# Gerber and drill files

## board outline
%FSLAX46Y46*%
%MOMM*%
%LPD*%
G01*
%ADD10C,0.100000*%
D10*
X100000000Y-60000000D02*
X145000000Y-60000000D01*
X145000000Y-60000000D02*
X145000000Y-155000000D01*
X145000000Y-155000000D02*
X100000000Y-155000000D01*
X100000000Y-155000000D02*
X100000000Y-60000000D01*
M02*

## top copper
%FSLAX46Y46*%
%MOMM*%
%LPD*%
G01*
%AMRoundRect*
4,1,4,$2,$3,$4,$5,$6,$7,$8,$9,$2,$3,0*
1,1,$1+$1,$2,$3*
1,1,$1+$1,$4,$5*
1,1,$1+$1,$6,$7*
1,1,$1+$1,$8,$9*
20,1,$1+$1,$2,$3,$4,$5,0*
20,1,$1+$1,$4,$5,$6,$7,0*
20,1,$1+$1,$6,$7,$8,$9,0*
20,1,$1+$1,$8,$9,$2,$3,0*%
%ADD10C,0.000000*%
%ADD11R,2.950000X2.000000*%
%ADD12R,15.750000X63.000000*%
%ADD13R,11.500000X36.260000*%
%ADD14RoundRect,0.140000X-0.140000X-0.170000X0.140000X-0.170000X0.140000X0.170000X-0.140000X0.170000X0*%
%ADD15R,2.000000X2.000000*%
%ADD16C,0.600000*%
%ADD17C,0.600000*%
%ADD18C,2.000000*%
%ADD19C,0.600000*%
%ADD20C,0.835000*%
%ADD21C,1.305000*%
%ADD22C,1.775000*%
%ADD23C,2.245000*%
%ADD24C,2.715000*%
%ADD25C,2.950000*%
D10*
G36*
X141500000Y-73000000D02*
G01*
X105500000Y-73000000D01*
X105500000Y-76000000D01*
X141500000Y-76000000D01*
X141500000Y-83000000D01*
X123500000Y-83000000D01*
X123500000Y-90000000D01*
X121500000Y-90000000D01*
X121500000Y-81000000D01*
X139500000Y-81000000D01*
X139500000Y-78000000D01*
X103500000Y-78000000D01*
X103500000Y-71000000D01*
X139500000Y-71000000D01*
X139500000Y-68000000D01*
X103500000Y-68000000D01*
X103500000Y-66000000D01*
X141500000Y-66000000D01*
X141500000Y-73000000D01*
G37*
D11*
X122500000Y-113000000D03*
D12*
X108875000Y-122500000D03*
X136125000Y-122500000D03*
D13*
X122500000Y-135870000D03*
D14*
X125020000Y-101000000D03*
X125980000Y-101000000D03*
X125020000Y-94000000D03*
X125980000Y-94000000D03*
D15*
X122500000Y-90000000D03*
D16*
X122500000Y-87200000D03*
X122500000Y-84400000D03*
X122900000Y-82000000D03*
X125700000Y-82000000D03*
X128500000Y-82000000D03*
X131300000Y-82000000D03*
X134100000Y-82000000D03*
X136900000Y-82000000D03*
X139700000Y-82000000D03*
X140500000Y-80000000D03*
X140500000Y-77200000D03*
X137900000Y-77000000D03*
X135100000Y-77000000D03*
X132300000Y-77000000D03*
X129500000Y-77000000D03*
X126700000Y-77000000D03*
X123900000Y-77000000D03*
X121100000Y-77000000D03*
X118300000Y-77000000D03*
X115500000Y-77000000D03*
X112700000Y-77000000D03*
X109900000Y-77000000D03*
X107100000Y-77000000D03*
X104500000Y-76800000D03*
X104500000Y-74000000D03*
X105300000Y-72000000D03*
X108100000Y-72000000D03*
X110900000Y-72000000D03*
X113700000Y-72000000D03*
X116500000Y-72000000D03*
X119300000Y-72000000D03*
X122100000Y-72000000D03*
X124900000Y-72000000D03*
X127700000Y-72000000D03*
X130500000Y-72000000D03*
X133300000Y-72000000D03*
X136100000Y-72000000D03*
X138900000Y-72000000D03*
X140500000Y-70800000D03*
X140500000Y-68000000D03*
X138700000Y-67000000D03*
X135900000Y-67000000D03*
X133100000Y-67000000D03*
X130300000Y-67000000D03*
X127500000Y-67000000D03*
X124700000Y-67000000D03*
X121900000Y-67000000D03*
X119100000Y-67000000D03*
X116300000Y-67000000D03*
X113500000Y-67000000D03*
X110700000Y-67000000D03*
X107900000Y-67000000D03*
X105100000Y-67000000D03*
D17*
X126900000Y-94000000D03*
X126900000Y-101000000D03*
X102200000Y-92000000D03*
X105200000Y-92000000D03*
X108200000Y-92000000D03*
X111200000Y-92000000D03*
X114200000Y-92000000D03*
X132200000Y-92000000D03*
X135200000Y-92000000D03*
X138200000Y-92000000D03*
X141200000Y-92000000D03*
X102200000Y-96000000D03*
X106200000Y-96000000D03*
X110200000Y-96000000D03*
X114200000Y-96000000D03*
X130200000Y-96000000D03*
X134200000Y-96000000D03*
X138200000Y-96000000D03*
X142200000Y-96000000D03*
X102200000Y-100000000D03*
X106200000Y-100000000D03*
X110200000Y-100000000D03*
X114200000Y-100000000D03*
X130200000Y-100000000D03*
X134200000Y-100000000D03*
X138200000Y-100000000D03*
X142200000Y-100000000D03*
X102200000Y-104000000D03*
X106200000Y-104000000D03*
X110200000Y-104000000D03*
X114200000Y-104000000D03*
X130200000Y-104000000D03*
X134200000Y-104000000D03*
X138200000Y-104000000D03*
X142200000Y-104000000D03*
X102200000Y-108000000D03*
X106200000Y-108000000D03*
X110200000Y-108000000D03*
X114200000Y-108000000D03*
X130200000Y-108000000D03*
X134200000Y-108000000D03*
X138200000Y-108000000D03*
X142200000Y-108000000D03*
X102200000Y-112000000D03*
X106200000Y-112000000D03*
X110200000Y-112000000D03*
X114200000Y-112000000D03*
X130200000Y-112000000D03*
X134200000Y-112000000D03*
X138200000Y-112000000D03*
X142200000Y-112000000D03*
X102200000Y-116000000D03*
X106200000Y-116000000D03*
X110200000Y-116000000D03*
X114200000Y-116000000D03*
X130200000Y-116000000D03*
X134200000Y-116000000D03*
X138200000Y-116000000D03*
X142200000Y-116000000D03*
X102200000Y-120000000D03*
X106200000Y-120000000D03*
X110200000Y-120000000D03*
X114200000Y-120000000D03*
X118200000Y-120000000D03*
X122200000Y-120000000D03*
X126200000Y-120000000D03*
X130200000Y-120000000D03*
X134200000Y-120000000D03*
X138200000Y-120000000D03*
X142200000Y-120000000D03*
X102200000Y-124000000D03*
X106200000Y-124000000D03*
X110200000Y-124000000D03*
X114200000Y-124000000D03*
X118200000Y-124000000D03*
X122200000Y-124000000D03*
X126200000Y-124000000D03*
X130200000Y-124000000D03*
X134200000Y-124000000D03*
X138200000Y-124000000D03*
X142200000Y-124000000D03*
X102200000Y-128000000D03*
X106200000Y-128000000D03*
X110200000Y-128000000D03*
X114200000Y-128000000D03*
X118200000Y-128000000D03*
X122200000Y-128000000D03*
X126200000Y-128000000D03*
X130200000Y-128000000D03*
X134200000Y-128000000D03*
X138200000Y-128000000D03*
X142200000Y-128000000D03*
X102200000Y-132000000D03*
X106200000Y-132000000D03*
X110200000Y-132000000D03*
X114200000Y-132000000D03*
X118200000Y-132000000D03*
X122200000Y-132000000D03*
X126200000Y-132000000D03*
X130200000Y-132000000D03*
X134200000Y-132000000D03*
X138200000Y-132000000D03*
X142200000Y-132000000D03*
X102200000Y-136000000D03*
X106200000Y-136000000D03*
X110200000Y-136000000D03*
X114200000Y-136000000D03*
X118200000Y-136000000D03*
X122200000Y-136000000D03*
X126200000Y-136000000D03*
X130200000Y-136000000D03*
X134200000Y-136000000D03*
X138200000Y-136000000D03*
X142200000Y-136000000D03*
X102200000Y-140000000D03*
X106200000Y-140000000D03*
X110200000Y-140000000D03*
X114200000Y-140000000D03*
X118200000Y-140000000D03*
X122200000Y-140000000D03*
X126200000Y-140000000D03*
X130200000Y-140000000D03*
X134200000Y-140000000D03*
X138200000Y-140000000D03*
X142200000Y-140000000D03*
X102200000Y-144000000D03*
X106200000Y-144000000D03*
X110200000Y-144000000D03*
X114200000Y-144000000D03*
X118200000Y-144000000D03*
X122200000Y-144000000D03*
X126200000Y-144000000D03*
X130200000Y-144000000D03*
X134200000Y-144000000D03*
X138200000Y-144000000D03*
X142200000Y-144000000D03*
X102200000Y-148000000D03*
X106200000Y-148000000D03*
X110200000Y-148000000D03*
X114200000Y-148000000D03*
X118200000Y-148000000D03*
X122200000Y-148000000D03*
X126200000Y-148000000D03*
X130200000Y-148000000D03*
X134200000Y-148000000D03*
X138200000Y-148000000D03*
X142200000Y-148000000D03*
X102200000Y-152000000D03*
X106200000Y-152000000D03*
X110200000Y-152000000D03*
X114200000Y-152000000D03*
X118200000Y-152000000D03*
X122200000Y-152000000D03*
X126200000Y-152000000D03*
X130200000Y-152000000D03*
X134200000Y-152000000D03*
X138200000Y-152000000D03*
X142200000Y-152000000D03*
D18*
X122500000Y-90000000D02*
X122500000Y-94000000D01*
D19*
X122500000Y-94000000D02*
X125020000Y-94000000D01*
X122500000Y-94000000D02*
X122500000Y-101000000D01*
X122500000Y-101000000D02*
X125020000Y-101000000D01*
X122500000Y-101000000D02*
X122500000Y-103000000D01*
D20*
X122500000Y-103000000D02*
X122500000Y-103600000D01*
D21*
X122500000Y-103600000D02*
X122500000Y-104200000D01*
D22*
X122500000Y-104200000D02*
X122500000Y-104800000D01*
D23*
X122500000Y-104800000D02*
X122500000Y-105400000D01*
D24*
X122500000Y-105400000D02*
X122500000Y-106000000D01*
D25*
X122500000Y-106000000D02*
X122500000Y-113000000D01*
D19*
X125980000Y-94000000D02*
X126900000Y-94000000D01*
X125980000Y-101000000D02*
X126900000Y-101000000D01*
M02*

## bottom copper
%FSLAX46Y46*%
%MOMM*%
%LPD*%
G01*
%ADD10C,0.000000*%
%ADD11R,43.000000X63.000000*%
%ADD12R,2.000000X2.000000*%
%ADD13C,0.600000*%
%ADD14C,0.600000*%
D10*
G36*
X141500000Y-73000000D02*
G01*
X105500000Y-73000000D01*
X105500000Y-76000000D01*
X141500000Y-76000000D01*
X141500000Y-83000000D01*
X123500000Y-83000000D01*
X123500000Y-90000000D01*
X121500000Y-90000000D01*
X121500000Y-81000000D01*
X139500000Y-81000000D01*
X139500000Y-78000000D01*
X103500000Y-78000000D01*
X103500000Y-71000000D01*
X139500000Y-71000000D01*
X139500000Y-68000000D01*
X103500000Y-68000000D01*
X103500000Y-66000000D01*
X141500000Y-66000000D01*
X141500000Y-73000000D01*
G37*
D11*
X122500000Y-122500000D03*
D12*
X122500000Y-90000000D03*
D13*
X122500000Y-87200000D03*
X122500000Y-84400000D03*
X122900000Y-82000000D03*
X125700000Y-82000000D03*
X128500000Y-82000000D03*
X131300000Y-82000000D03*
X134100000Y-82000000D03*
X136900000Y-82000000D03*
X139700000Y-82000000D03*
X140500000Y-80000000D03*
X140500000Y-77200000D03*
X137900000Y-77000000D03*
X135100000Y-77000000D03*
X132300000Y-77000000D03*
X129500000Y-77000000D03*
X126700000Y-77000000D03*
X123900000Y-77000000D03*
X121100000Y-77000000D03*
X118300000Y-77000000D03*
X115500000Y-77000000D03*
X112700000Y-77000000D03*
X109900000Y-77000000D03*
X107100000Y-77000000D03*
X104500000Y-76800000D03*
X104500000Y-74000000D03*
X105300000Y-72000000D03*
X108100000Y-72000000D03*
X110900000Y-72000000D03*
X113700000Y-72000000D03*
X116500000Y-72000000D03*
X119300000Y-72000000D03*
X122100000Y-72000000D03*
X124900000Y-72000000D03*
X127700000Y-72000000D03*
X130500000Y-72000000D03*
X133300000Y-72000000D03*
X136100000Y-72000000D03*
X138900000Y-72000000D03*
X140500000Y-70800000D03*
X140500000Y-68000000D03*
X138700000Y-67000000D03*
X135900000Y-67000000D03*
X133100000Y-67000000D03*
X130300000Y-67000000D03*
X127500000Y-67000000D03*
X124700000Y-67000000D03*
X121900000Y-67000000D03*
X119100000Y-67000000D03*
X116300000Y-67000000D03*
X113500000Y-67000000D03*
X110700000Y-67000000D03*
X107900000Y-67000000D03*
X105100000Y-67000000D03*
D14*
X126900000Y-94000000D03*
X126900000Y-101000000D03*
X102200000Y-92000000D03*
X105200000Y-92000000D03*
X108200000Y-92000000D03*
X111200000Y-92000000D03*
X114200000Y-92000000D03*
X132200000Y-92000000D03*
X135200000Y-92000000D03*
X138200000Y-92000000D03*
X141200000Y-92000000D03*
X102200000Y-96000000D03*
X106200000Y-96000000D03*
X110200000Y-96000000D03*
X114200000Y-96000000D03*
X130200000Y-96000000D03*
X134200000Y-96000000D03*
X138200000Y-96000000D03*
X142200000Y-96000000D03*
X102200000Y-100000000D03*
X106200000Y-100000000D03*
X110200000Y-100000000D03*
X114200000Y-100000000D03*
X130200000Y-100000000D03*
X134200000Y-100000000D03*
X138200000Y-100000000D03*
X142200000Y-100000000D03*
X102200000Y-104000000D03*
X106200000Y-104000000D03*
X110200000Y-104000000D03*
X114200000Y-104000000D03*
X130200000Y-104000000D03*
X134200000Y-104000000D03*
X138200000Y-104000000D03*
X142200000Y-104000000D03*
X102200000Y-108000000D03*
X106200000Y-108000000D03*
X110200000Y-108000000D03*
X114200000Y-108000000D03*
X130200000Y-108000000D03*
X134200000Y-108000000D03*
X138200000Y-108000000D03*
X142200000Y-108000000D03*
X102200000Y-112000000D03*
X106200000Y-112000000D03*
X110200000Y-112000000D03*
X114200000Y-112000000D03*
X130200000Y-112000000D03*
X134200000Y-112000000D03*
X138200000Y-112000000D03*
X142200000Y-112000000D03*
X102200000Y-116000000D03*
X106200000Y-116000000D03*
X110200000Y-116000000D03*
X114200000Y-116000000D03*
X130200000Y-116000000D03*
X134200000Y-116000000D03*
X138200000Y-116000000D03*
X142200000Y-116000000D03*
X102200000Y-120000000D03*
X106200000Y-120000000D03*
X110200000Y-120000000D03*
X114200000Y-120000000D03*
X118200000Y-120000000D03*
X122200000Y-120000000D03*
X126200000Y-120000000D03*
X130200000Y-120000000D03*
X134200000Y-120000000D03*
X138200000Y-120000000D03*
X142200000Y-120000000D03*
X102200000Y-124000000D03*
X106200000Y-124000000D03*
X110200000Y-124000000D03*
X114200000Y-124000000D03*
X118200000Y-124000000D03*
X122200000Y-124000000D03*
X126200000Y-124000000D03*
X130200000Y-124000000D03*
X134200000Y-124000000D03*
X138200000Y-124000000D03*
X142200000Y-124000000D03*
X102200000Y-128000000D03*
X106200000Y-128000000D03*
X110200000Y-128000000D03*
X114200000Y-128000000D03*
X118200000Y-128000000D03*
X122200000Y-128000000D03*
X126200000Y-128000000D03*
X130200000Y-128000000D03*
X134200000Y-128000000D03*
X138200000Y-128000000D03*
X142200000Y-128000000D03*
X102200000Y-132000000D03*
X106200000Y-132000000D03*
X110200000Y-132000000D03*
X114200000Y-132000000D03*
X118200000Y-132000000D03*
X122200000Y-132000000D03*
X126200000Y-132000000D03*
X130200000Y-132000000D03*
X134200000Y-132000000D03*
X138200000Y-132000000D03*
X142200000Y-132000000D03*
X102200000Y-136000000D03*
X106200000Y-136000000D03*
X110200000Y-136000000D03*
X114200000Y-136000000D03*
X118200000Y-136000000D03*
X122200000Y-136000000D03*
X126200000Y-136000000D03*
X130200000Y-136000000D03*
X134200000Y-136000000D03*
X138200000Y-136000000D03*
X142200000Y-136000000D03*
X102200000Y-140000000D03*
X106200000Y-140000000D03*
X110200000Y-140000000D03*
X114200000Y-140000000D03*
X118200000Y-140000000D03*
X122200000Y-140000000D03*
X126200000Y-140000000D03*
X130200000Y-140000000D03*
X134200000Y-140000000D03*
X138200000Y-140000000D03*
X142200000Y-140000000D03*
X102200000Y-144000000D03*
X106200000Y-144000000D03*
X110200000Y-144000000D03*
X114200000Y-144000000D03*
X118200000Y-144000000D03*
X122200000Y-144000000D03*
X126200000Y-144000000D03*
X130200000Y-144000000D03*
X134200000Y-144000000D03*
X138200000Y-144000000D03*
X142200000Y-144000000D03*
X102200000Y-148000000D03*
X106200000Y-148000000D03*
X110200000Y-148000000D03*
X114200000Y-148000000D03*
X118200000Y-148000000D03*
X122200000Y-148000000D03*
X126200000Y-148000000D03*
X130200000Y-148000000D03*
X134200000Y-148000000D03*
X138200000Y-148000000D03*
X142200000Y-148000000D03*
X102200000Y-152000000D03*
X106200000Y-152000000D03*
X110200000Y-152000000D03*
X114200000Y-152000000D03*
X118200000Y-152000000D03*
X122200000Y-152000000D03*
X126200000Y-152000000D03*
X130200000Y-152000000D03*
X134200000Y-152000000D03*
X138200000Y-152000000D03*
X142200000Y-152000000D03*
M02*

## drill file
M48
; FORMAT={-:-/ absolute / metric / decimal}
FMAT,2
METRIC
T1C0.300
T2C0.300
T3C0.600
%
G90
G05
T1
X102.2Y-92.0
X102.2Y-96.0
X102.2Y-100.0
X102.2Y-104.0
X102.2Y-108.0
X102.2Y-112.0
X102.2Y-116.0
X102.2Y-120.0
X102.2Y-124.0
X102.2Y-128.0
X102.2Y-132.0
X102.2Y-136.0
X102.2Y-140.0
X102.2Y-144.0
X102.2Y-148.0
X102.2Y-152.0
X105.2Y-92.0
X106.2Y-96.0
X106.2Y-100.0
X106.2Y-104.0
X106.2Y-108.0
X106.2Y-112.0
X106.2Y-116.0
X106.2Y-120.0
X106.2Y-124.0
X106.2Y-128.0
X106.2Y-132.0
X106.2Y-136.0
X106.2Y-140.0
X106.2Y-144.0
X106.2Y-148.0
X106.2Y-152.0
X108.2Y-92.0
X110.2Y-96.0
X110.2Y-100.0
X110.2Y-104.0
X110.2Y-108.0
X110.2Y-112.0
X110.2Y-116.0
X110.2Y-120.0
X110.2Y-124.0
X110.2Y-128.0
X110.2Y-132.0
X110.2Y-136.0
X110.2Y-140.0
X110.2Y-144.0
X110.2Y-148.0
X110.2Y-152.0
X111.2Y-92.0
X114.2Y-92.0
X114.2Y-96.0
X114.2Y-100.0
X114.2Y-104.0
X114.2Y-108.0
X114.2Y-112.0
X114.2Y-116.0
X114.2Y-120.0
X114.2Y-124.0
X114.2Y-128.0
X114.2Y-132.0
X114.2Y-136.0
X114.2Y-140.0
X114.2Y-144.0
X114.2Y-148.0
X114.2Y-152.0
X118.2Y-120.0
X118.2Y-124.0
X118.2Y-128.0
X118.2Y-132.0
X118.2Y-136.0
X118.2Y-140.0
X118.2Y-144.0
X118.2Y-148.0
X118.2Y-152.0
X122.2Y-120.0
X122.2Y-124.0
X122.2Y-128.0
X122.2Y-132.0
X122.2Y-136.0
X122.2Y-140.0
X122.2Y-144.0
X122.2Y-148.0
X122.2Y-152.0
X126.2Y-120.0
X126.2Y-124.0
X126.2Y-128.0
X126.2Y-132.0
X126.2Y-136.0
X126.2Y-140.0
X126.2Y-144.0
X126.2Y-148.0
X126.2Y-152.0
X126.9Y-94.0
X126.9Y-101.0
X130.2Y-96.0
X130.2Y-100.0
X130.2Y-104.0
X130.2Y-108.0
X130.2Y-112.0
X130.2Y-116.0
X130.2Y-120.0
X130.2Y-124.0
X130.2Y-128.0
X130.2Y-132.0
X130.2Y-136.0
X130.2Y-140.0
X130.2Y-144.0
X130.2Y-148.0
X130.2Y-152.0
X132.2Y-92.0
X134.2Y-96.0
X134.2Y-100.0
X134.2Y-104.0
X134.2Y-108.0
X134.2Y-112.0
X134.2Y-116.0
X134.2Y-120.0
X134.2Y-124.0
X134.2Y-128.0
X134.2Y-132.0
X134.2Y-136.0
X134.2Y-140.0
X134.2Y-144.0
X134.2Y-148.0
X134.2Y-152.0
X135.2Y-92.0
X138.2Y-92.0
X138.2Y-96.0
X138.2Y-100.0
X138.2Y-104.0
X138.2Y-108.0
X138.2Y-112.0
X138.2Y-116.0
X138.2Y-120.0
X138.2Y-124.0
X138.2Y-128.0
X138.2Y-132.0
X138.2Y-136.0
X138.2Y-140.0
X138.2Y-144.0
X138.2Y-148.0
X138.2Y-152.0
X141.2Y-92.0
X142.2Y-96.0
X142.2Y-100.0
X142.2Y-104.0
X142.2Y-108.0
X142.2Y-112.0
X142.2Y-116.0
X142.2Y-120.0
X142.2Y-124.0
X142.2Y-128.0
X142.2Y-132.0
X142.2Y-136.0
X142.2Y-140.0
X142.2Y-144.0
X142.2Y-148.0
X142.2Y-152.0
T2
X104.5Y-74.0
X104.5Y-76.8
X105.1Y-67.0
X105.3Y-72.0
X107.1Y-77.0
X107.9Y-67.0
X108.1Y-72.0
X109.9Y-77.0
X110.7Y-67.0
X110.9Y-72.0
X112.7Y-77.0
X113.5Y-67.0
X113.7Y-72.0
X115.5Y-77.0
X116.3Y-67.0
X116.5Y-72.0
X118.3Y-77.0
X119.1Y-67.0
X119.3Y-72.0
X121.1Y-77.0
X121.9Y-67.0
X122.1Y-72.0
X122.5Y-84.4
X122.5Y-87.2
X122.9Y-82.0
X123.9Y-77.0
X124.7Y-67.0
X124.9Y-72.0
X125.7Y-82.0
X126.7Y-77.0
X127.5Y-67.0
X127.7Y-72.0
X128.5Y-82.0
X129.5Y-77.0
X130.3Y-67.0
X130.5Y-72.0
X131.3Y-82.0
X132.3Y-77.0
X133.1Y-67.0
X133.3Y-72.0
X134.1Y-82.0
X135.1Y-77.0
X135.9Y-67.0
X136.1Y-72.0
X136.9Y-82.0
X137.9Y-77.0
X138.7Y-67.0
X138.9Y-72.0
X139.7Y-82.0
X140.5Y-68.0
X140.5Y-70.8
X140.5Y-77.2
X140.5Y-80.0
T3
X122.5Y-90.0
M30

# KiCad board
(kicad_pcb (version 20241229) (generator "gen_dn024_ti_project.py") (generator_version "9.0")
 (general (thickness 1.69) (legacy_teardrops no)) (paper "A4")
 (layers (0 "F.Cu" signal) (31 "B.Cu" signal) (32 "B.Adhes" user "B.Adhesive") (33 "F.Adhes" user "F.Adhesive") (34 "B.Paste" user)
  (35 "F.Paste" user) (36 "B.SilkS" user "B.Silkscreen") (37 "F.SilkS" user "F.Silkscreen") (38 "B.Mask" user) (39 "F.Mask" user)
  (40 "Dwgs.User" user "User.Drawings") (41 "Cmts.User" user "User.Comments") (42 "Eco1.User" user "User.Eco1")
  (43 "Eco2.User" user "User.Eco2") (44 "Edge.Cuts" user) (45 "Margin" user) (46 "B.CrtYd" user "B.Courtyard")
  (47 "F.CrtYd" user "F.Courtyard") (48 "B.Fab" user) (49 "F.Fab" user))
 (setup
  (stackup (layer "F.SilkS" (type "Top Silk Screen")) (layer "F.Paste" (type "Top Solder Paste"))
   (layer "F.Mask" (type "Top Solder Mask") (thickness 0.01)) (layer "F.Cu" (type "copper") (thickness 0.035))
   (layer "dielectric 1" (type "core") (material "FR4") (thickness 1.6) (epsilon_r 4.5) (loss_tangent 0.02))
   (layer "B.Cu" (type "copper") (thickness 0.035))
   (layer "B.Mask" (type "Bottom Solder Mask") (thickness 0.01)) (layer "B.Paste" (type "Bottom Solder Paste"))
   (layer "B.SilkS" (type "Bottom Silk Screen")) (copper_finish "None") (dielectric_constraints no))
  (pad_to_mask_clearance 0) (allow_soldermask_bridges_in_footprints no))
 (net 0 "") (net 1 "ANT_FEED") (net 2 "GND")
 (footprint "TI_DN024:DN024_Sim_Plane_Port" (layer "F.Cu") (at 122.5 113)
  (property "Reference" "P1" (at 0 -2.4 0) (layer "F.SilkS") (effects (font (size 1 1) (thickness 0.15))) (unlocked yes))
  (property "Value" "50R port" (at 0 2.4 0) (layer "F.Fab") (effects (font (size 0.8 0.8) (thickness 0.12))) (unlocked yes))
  (pad "1" smd rect (at 0 0) (size 2.95 2) (layers "F.Cu" "F.Mask") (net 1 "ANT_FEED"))
  (pad "2" smd rect (at 0 9.5) (size 43 63) (layers "B.Cu" "B.Mask") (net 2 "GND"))
  (pad "2" smd rect (at -13.625 9.5) (size 15.75 63) (layers "F.Cu" "F.Mask") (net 2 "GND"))
  (pad "2" smd rect (at 13.625 9.5) (size 15.75 63) (layers "F.Cu" "F.Mask") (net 2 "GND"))
  (pad "2" smd rect (at 0 22.87) (size 11.5 36.26) (layers "F.Cu" "F.Mask") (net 2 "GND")))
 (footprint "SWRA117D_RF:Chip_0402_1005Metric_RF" (layer "F.Cu") (at 125.5 101)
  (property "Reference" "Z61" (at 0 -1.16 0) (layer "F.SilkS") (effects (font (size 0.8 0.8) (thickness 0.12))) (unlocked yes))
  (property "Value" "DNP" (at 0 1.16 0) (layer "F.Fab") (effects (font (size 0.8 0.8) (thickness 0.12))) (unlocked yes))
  (pad "1" smd roundrect (at -0.48 0) (size 0.56 0.62) (layers "F.Cu" "F.Paste" "F.Mask") (roundrect_rratio 0.25) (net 1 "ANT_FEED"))
  (pad "2" smd roundrect (at 0.48 0) (size 0.56 0.62) (layers "F.Cu" "F.Paste" "F.Mask") (roundrect_rratio 0.25) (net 2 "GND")))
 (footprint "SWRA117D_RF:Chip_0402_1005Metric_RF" (layer "F.Cu") (at 125.5 94)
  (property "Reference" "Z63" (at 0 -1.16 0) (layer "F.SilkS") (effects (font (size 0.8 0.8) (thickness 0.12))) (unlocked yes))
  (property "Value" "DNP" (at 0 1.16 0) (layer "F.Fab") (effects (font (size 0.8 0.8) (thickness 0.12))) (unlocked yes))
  (pad "1" smd roundrect (at -0.48 0) (size 0.56 0.62) (layers "F.Cu" "F.Paste" "F.Mask") (roundrect_rratio 0.25) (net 1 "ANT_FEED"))
  (pad "2" smd roundrect (at 0.48 0) (size 0.56 0.62) (layers "F.Cu" "F.Paste" "F.Mask") (roundrect_rratio 0.25) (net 2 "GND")))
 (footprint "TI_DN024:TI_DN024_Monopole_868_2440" (layer "F.Cu") (at 122.5 90)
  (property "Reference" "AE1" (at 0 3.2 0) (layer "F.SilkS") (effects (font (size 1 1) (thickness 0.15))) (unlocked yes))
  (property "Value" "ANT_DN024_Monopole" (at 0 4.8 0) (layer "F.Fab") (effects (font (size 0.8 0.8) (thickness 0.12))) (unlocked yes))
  (fp_poly
   (pts (xy 1 0) (xy 1 -7) (xy 19 -7) (xy 19 -14) (xy -17 -14) (xy -17 -17) (xy 19 -17) (xy 19 -24) (xy -19 -24) (xy -19 -22) (xy 17 -22)
    (xy 17 -19) (xy -19 -19) (xy -19 -12) (xy 17 -12) (xy 17 -9) (xy -1 -9) (xy -1 0))
   (stroke (width 0) (type solid)) (fill yes) (layer "F.Cu"))
  (fp_poly
   (pts (xy 1 0) (xy 1 -7) (xy 19 -7) (xy 19 -14) (xy -17 -14) (xy -17 -17) (xy 19 -17) (xy 19 -24) (xy -19 -24) (xy -19 -22) (xy 17 -22)
    (xy 17 -19) (xy -19 -19) (xy -19 -12) (xy 17 -12) (xy 17 -9) (xy -1 -9) (xy -1 0))
   (stroke (width 0) (type solid)) (fill yes) (layer "B.Cu"))
  (pad "1" thru_hole rect (at 0 0) (size 2 2) (drill 0.6) (layers "*.Cu" "*.Mask") (remove_unused_layers no) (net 1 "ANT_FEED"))
  (pad "1" thru_hole circle (at 0 -2.8) (size 0.6 0.6) (drill 0.3) (layers "*.Cu") (remove_unused_layers no) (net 1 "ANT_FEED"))
  (pad "1" thru_hole circle (at 0 -5.6) (size 0.6 0.6) (drill 0.3) (layers "*.Cu") (remove_unused_layers no) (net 1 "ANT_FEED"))
  (pad "1" thru_hole circle (at 0.4 -8) (size 0.6 0.6) (drill 0.3) (layers "*.Cu") (remove_unused_layers no) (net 1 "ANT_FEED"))
  (pad "1" thru_hole circle (at 3.2 -8) (size 0.6 0.6) (drill 0.3) (layers "*.Cu") (remove_unused_layers no) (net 1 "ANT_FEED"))
  (pad "1" thru_hole circle (at 6 -8) (size 0.6 0.6) (drill 0.3) (layers "*.Cu") (remove_unused_layers no) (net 1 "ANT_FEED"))
  (pad "1" thru_hole circle (at 8.8 -8) (size 0.6 0.6) (drill 0.3) (layers "*.Cu") (remove_unused_layers no) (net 1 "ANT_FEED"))
  (pad "1" thru_hole circle (at 11.6 -8) (size 0.6 0.6) (drill 0.3) (layers "*.Cu") (remove_unused_layers no) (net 1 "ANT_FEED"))
  (pad "1" thru_hole circle (at 14.4 -8) (size 0.6 0.6) (drill 0.3) (layers "*.Cu") (remove_unused_layers no) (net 1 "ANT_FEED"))
  (pad "1" thru_hole circle (at 17.2 -8) (size 0.6 0.6) (drill 0.3) (layers "*.Cu") (remove_unused_layers no) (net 1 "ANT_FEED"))
  (pad "1" thru_hole circle (at 18 -10) (size 0.6 0.6) (drill 0.3) (layers "*.Cu") (remove_unused_layers no) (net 1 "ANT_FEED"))
  (pad "1" thru_hole circle (at 18 -12.8) (size 0.6 0.6) (drill 0.3) (layers "*.Cu") (remove_unused_layers no) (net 1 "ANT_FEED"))
  (pad "1" thru_hole circle (at 15.4 -13) (size 0.6 0.6) (drill 0.3) (layers "*.Cu") (remove_unused_layers no) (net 1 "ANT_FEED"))
  (pad "1" thru_hole circle (at 12.6 -13) (size 0.6 0.6) (drill 0.3) (layers "*.Cu") (remove_unused_layers no) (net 1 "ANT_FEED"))
  (pad "1" thru_hole circle (at 9.8 -13) (size 0.6 0.6) (drill 0.3) (layers "*.Cu") (remove_unused_layers no) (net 1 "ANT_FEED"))
  (pad "1" thru_hole circle (at 7 -13) (size 0.6 0.6) (drill 0.3) (layers "*.Cu") (remove_unused_layers no) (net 1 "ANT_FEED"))
  (pad "1" thru_hole circle (at 4.2 -13) (size 0.6 0.6) (drill 0.3) (layers "*.Cu") (remove_unused_layers no) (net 1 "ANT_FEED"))
  (pad "1" thru_hole circle (at 1.4 -13) (size 0.6 0.6) (drill 0.3) (layers "*.Cu") (remove_unused_layers no) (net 1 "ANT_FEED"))
  (pad "1" thru_hole circle (at -1.4 -13) (size 0.6 0.6) (drill 0.3) (layers "*.Cu") (remove_unused_layers no) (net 1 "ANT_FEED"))
  (pad "1" thru_hole circle (at -4.2 -13) (size 0.6 0.6) (drill 0.3) (layers "*.Cu") (remove_unused_layers no) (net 1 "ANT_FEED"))
  (pad "1" thru_hole circle (at -7 -13) (size 0.6 0.6) (drill 0.3) (layers "*.Cu") (remove_unused_layers no) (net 1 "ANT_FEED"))
  (pad "1" thru_hole circle (at -9.8 -13) (size 0.6 0.6) (drill 0.3) (layers "*.Cu") (remove_unused_layers no) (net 1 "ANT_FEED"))
  (pad "1" thru_hole circle (at -12.6 -13) (size 0.6 0.6) (drill 0.3) (layers "*.Cu") (remove_unused_layers no) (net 1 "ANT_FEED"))
  (pad "1" thru_hole circle (at -15.4 -13) (size 0.6 0.6) (drill 0.3) (layers "*.Cu") (remove_unused_layers no) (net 1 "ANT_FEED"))
  (pad "1" thru_hole circle (at -18 -13.2) (size 0.6 0.6) (drill 0.3) (layers "*.Cu") (remove_unused_layers no) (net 1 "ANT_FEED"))
  (pad "1" thru_hole circle (at -18 -16) (size 0.6 0.6) (drill 0.3) (layers "*.Cu") (remove_unused_layers no) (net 1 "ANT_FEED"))
  (pad "1" thru_hole circle (at -17.2 -18) (size 0.6 0.6) (drill 0.3) (layers "*.Cu") (remove_unused_layers no) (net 1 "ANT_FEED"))
  (pad "1" thru_hole circle (at -14.4 -18) (size 0.6 0.6) (drill 0.3) (layers "*.Cu") (remove_unused_layers no) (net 1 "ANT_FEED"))
  (pad "1" thru_hole circle (at -11.6 -18) (size 0.6 0.6) (drill 0.3) (layers "*.Cu") (remove_unused_layers no) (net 1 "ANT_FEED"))
  (pad "1" thru_hole circle (at -8.8 -18) (size 0.6 0.6) (drill 0.3) (layers "*.Cu") (remove_unused_layers no) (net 1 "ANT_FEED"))
  (pad "1" thru_hole circle (at -6 -18) (size 0.6 0.6) (drill 0.3) (layers "*.Cu") (remove_unused_layers no) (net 1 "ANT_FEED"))
  (pad "1" thru_hole circle (at -3.2 -18) (size 0.6 0.6) (drill 0.3) (layers "*.Cu") (remove_unused_layers no) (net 1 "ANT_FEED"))
  (pad "1" thru_hole circle (at -0.4 -18) (size 0.6 0.6) (drill 0.3) (layers "*.Cu") (remove_unused_layers no) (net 1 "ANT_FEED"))
  (pad "1" thru_hole circle (at 2.4 -18) (size 0.6 0.6) (drill 0.3) (layers "*.Cu") (remove_unused_layers no) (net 1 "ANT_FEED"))
  (pad "1" thru_hole circle (at 5.2 -18) (size 0.6 0.6) (drill 0.3) (layers "*.Cu") (remove_unused_layers no) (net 1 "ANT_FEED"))
  (pad "1" thru_hole circle (at 8 -18) (size 0.6 0.6) (drill 0.3) (layers "*.Cu") (remove_unused_layers no) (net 1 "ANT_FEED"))
  (pad "1" thru_hole circle (at 10.8 -18) (size 0.6 0.6) (drill 0.3) (layers "*.Cu") (remove_unused_layers no) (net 1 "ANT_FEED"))
  (pad "1" thru_hole circle (at 13.6 -18) (size 0.6 0.6) (drill 0.3) (layers "*.Cu") (remove_unused_layers no) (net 1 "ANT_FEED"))
  (pad "1" thru_hole circle (at 16.4 -18) (size 0.6 0.6) (drill 0.3) (layers "*.Cu") (remove_unused_layers no) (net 1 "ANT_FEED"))
  (pad "1" thru_hole circle (at 18 -19.2) (size 0.6 0.6) (drill 0.3) (layers "*.Cu") (remove_unused_layers no) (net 1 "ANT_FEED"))
  (pad "1" thru_hole circle (at 18 -22) (size 0.6 0.6) (drill 0.3) (layers "*.Cu") (remove_unused_layers no) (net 1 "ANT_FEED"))
  (pad "1" thru_hole circle (at 16.2 -23) (size 0.6 0.6) (drill 0.3) (layers "*.Cu") (remove_unused_layers no) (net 1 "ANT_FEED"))
  (pad "1" thru_hole circle (at 13.4 -23) (size 0.6 0.6) (drill 0.3) (layers "*.Cu") (remove_unused_layers no) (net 1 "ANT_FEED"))
  (pad "1" thru_hole circle (at 10.6 -23) (size 0.6 0.6) (drill 0.3) (layers "*.Cu") (remove_unused_layers no) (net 1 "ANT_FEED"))
  (pad "1" thru_hole circle (at 7.8 -23) (size 0.6 0.6) (drill 0.3) (layers "*.Cu") (remove_unused_layers no) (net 1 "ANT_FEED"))
  (pad "1" thru_hole circle (at 5 -23) (size 0.6 0.6) (drill 0.3) (layers "*.Cu") (remove_unused_layers no) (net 1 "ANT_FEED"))
  (pad "1" thru_hole circle (at 2.2 -23) (size 0.6 0.6) (drill 0.3) (layers "*.Cu") (remove_unused_layers no) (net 1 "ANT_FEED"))
  (pad "1" thru_hole circle (at -0.6 -23) (size 0.6 0.6) (drill 0.3) (layers "*.Cu") (remove_unused_layers no) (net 1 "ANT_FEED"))
  (pad "1" thru_hole circle (at -3.4 -23) (size 0.6 0.6) (drill 0.3) (layers "*.Cu") (remove_unused_layers no) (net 1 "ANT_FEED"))
  (pad "1" thru_hole circle (at -6.2 -23) (size 0.6 0.6) (drill 0.3) (layers "*.Cu") (remove_unused_layers no) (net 1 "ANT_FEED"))
  (pad "1" thru_hole circle (at -9 -23) (size 0.6 0.6) (drill 0.3) (layers "*.Cu") (remove_unused_layers no) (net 1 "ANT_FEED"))
  (pad "1" thru_hole circle (at -11.8 -23) (size 0.6 0.6) (drill 0.3) (layers "*.Cu") (remove_unused_layers no) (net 1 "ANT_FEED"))
  (pad "1" thru_hole circle (at -14.6 -23) (size 0.6 0.6) (drill 0.3) (layers "*.Cu") (remove_unused_layers no) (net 1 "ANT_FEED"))
  (pad "1" thru_hole circle (at -17.4 -23) (size 0.6 0.6) (drill 0.3) (layers "*.Cu") (remove_unused_layers no) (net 1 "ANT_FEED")))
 (gr_line (start 100 60) (end 145 60) (stroke (width 0.1) (type solid)) (layer "Edge.Cuts"))
 (gr_line (start 145 60) (end 145 155) (stroke (width 0.1) (type solid)) (layer "Edge.Cuts"))
 (gr_line (start 145 155) (end 100 155) (stroke (width 0.1) (type solid)) (layer "Edge.Cuts"))
 (gr_line (start 100 155) (end 100 60) (stroke (width 0.1) (type solid)) (layer "Edge.Cuts"))
 (segment (start 122.5 90) (end 122.5 94) (width 2) (layer "F.Cu") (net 1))
 (segment (start 122.5 94) (end 125.02 94) (width 0.6) (layer "F.Cu") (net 1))
 (segment (start 122.5 94) (end 122.5 101) (width 0.6) (layer "F.Cu") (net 1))
 (segment (start 122.5 101) (end 125.02 101) (width 0.6) (layer "F.Cu") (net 1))
 (segment (start 122.5 101) (end 122.5 103) (width 0.6) (layer "F.Cu") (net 1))
 (segment (start 122.5 103) (end 122.5 103.6) (width 0.835) (layer "F.Cu") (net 1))
 (segment (start 122.5 103.6) (end 122.5 104.2) (width 1.305) (layer "F.Cu") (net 1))
 (segment (start 122.5 104.2) (end 122.5 104.8) (width 1.775) (layer "F.Cu") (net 1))
 (segment (start 122.5 104.8) (end 122.5 105.4) (width 2.245) (layer "F.Cu") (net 1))
 (segment (start 122.5 105.4) (end 122.5 106) (width 2.715) (layer "F.Cu") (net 1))
 (segment (start 122.5 106) (end 122.5 113) (width 2.95) (layer "F.Cu") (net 1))
 (segment (start 125.98 94) (end 126.9 94) (width 0.6) (layer "F.Cu") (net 2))
 (segment (start 125.98 101) (end 126.9 101) (width 0.6) (layer "F.Cu") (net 2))
 (via (at 126.9 94) (size 0.6) (drill 0.3) (layers "F.Cu" "B.Cu") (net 2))
 (via (at 126.9 101) (size 0.6) (drill 0.3) (layers "F.Cu" "B.Cu") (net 2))
 (via (at 102.2 92) (size 0.6) (drill 0.3) (layers "F.Cu" "B.Cu") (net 2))
 (via (at 105.2 92) (size 0.6) (drill 0.3) (layers "F.Cu" "B.Cu") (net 2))
 (via (at 108.2 92) (size 0.6) (drill 0.3) (layers "F.Cu" "B.Cu") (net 2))
 (via (at 111.2 92) (size 0.6) (drill 0.3) (layers "F.Cu" "B.Cu") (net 2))
 (via (at 114.2 92) (size 0.6) (drill 0.3) (layers "F.Cu" "B.Cu") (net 2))
 (via (at 132.2 92) (size 0.6) (drill 0.3) (layers "F.Cu" "B.Cu") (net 2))
 (via (at 135.2 92) (size 0.6) (drill 0.3) (layers "F.Cu" "B.Cu") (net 2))
 (via (at 138.2 92) (size 0.6) (drill 0.3) (layers "F.Cu" "B.Cu") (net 2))
 (via (at 141.2 92) (size 0.6) (drill 0.3) (layers "F.Cu" "B.Cu") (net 2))
 (via (at 102.2 96) (size 0.6) (drill 0.3) (layers "F.Cu" "B.Cu") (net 2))
 (via (at 106.2 96) (size 0.6) (drill 0.3) (layers "F.Cu" "B.Cu") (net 2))
 (via (at 110.2 96) (size 0.6) (drill 0.3) (layers "F.Cu" "B.Cu") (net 2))
 (via (at 114.2 96) (size 0.6) (drill 0.3) (layers "F.Cu" "B.Cu") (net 2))
 (via (at 130.2 96) (size 0.6) (drill 0.3) (layers "F.Cu" "B.Cu") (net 2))
 (via (at 134.2 96) (size 0.6) (drill 0.3) (layers "F.Cu" "B.Cu") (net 2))
 (via (at 138.2 96) (size 0.6) (drill 0.3) (layers "F.Cu" "B.Cu") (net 2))
 (via (at 142.2 96) (size 0.6) (drill 0.3) (layers "F.Cu" "B.Cu") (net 2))
 (via (at 102.2 100) (size 0.6) (drill 0.3) (layers "F.Cu" "B.Cu") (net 2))
 (via (at 106.2 100) (size 0.6) (drill 0.3) (layers "F.Cu" "B.Cu") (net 2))
 (via (at 110.2 100) (size 0.6) (drill 0.3) (layers "F.Cu" "B.Cu") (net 2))
 (via (at 114.2 100) (size 0.6) (drill 0.3) (layers "F.Cu" "B.Cu") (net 2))
 (via (at 130.2 100) (size 0.6) (drill 0.3) (layers "F.Cu" "B.Cu") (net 2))
 (via (at 134.2 100) (size 0.6) (drill 0.3) (layers "F.Cu" "B.Cu") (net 2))
 (via (at 138.2 100) (size 0.6) (drill 0.3) (layers "F.Cu" "B.Cu") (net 2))
 (via (at 142.2 100) (size 0.6) (drill 0.3) (layers "F.Cu" "B.Cu") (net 2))
 (via (at 102.2 104) (size 0.6) (drill 0.3) (layers "F.Cu" "B.Cu") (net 2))
 (via (at 106.2 104) (size 0.6) (drill 0.3) (layers "F.Cu" "B.Cu") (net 2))
 (via (at 110.2 104) (size 0.6) (drill 0.3) (layers "F.Cu" "B.Cu") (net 2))
 (via (at 114.2 104) (size 0.6) (drill 0.3) (layers "F.Cu" "B.Cu") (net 2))
 (via (at 130.2 104) (size 0.6) (drill 0.3) (layers "F.Cu" "B.Cu") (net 2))
 (via (at 134.2 104) (size 0.6) (drill 0.3) (layers "F.Cu" "B.Cu") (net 2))
 (via (at 138.2 104) (size 0.6) (drill 0.3) (layers "F.Cu" "B.Cu") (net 2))
 (via (at 142.2 104) (size 0.6) (drill 0.3) (layers "F.Cu" "B.Cu") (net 2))
 (via (at 102.2 108) (size 0.6) (drill 0.3) (layers "F.Cu" "B.Cu") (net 2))
 (via (at 106.2 108) (size 0.6) (drill 0.3) (layers "F.Cu" "B.Cu") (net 2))
 (via (at 110.2 108) (size 0.6) (drill 0.3) (layers "F.Cu" "B.Cu") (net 2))
 (via (at 114.2 108) (size 0.6) (drill 0.3) (layers "F.Cu" "B.Cu") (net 2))
 (via (at 130.2 108) (size 0.6) (drill 0.3) (layers "F.Cu" "B.Cu") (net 2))
 (via (at 134.2 108) (size 0.6) (drill 0.3) (layers "F.Cu" "B.Cu") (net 2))
 (via (at 138.2 108) (size 0.6) (drill 0.3) (layers "F.Cu" "B.Cu") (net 2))
 (via (at 142.2 108) (size 0.6) (drill 0.3) (layers "F.Cu" "B.Cu") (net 2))
 (via (at 102.2 112) (size 0.6) (drill 0.3) (layers "F.Cu" "B.Cu") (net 2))
 (via (at 106.2 112) (size 0.6) (drill 0.3) (layers "F.Cu" "B.Cu") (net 2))
 (via (at 110.2 112) (size 0.6) (drill 0.3) (layers "F.Cu" "B.Cu") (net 2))
 (via (at 114.2 112) (size 0.6) (drill 0.3) (layers "F.Cu" "B.Cu") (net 2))
 (via (at 130.2 112) (size 0.6) (drill 0.3) (layers "F.Cu" "B.Cu") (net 2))
 (via (at 134.2 112) (size 0.6) (drill 0.3) (layers "F.Cu" "B.Cu") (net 2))
 (via (at 138.2 112) (size 0.6) (drill 0.3) (layers "F.Cu" "B.Cu") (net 2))
 (via (at 142.2 112) (size 0.6) (drill 0.3) (layers "F.Cu" "B.Cu") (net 2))
 (via (at 102.2 116) (size 0.6) (drill 0.3) (layers "F.Cu" "B.Cu") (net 2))
 (via (at 106.2 116) (size 0.6) (drill 0.3) (layers "F.Cu" "B.Cu") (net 2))
 (via (at 110.2 116) (size 0.6) (drill 0.3) (layers "F.Cu" "B.Cu") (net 2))
 (via (at 114.2 116) (size 0.6) (drill 0.3) (layers "F.Cu" "B.Cu") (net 2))
 (via (at 130.2 116) (size 0.6) (drill 0.3) (layers "F.Cu" "B.Cu") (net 2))
 (via (at 134.2 116) (size 0.6) (drill 0.3) (layers "F.Cu" "B.Cu") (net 2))
 (via (at 138.2 116) (size 0.6) (drill 0.3) (layers "F.Cu" "B.Cu") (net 2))
 (via (at 142.2 116) (size 0.6) (drill 0.3) (layers "F.Cu" "B.Cu") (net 2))
 (via (at 102.2 120) (size 0.6) (drill 0.3) (layers "F.Cu" "B.Cu") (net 2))
 (via (at 106.2 120) (size 0.6) (drill 0.3) (layers "F.Cu" "B.Cu") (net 2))
 (via (at 110.2 120) (size 0.6) (drill 0.3) (layers "F.Cu" "B.Cu") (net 2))
 (via (at 114.2 120) (size 0.6) (drill 0.3) (layers "F.Cu" "B.Cu") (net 2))
 (via (at 118.2 120) (size 0.6) (drill 0.3) (layers "F.Cu" "B.Cu") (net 2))
 (via (at 122.2 120) (size 0.6) (drill 0.3) (layers "F.Cu" "B.Cu") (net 2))
 (via (at 126.2 120) (size 0.6) (drill 0.3) (layers "F.Cu" "B.Cu") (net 2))
 (via (at 130.2 120) (size 0.6) (drill 0.3) (layers "F.Cu" "B.Cu") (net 2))
 (via (at 134.2 120) (size 0.6) (drill 0.3) (layers "F.Cu" "B.Cu") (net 2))
 (via (at 138.2 120) (size 0.6) (drill 0.3) (layers "F.Cu" "B.Cu") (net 2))
 (via (at 142.2 120) (size 0.6) (drill 0.3) (layers "F.Cu" "B.Cu") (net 2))
 (via (at 102.2 124) (size 0.6) (drill 0.3) (layers "F.Cu" "B.Cu") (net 2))
 (via (at 106.2 124) (size 0.6) (drill 0.3) (layers "F.Cu" "B.Cu") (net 2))
 (via (at 110.2 124) (size 0.6) (drill 0.3) (layers "F.Cu" "B.Cu") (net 2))
 (via (at 114.2 124) (size 0.6) (drill 0.3) (layers "F.Cu" "B.Cu") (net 2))
 (via (at 118.2 124) (size 0.6) (drill 0.3) (layers "F.Cu" "B.Cu") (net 2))
 (via (at 122.2 124) (size 0.6) (drill 0.3) (layers "F.Cu" "B.Cu") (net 2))
 (via (at 126.2 124) (size 0.6) (drill 0.3) (layers "F.Cu" "B.Cu") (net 2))
 (via (at 130.2 124) (size 0.6) (drill 0.3) (layers "F.Cu" "B.Cu") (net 2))
 (via (at 134.2 124) (size 0.6) (drill 0.3) (layers "F.Cu" "B.Cu") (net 2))
 (via (at 138.2 124) (size 0.6) (drill 0.3) (layers "F.Cu" "B.Cu") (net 2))
 (via (at 142.2 124) (size 0.6) (drill 0.3) (layers "F.Cu" "B.Cu") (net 2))
 (via (at 102.2 128) (size 0.6) (drill 0.3) (layers "F.Cu" "B.Cu") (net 2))
 (via (at 106.2 128) (size 0.6) (drill 0.3) (layers "F.Cu" "B.Cu") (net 2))
 (via (at 110.2 128) (size 0.6) (drill 0.3) (layers "F.Cu" "B.Cu") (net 2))
 (via (at 114.2 128) (size 0.6) (drill 0.3) (layers "F.Cu" "B.Cu") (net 2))
 (via (at 118.2 128) (size 0.6) (drill 0.3) (layers "F.Cu" "B.Cu") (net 2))
 (via (at 122.2 128) (size 0.6) (drill 0.3) (layers "F.Cu" "B.Cu") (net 2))
 (via (at 126.2 128) (size 0.6) (drill 0.3) (layers "F.Cu" "B.Cu") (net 2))
 (via (at 130.2 128) (size 0.6) (drill 0.3) (layers "F.Cu" "B.Cu") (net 2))
 (via (at 134.2 128) (size 0.6) (drill 0.3) (layers "F.Cu" "B.Cu") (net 2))
 (via (at 138.2 128) (size 0.6) (drill 0.3) (layers "F.Cu" "B.Cu") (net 2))
 (via (at 142.2 128) (size 0.6) (drill 0.3) (layers "F.Cu" "B.Cu") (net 2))
 (via (at 102.2 132) (size 0.6) (drill 0.3) (layers "F.Cu" "B.Cu") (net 2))
 (via (at 106.2 132) (size 0.6) (drill 0.3) (layers "F.Cu" "B.Cu") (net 2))
 (via (at 110.2 132) (size 0.6) (drill 0.3) (layers "F.Cu" "B.Cu") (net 2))
 (via (at 114.2 132) (size 0.6) (drill 0.3) (layers "F.Cu" "B.Cu") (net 2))
 (via (at 118.2 132) (size 0.6) (drill 0.3) (layers "F.Cu" "B.Cu") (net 2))
 (via (at 122.2 132) (size 0.6) (drill 0.3) (layers "F.Cu" "B.Cu") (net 2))
 (via (at 126.2 132) (size 0.6) (drill 0.3) (layers "F.Cu" "B.Cu") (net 2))
 (via (at 130.2 132) (size 0.6) (drill 0.3) (layers "F.Cu" "B.Cu") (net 2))
 (via (at 134.2 132) (size 0.6) (drill 0.3) (layers "F.Cu" "B.Cu") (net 2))
 (via (at 138.2 132) (size 0.6) (drill 0.3) (layers "F.Cu" "B.Cu") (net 2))
 (via (at 142.2 132) (size 0.6) (drill 0.3) (layers "F.Cu" "B.Cu") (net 2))
 (via (at 102.2 136) (size 0.6) (drill 0.3) (layers "F.Cu" "B.Cu") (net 2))
 (via (at 106.2 136) (size 0.6) (drill 0.3) (layers "F.Cu" "B.Cu") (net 2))
 (via (at 110.2 136) (size 0.6) (drill 0.3) (layers "F.Cu" "B.Cu") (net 2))
 (via (at 114.2 136) (size 0.6) (drill 0.3) (layers "F.Cu" "B.Cu") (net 2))
 (via (at 118.2 136) (size 0.6) (drill 0.3) (layers "F.Cu" "B.Cu") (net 2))
 (via (at 122.2 136) (size 0.6) (drill 0.3) (layers "F.Cu" "B.Cu") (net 2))
 (via (at 126.2 136) (size 0.6) (drill 0.3) (layers "F.Cu" "B.Cu") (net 2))
 (via (at 130.2 136) (size 0.6) (drill 0.3) (layers "F.Cu" "B.Cu") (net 2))
 (via (at 134.2 136) (size 0.6) (drill 0.3) (layers "F.Cu" "B.Cu") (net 2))
 (via (at 138.2 136) (size 0.6) (drill 0.3) (layers "F.Cu" "B.Cu") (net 2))
 (via (at 142.2 136) (size 0.6) (drill 0.3) (layers "F.Cu" "B.Cu") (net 2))
 (via (at 102.2 140) (size 0.6) (drill 0.3) (layers "F.Cu" "B.Cu") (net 2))
 (via (at 106.2 140) (size 0.6) (drill 0.3) (layers "F.Cu" "B.Cu") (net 2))
 (via (at 110.2 140) (size 0.6) (drill 0.3) (layers "F.Cu" "B.Cu") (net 2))
 (via (at 114.2 140) (size 0.6) (drill 0.3) (layers "F.Cu" "B.Cu") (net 2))
 (via (at 118.2 140) (size 0.6) (drill 0.3) (layers "F.Cu" "B.Cu") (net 2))
 (via (at 122.2 140) (size 0.6) (drill 0.3) (layers "F.Cu" "B.Cu") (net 2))
 (via (at 126.2 140) (size 0.6) (drill 0.3) (layers "F.Cu" "B.Cu") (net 2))
 (via (at 130.2 140) (size 0.6) (drill 0.3) (layers "F.Cu" "B.Cu") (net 2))
 (via (at 134.2 140) (size 0.6) (drill 0.3) (layers "F.Cu" "B.Cu") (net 2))
 (via (at 138.2 140) (size 0.6) (drill 0.3) (layers "F.Cu" "B.Cu") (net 2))
 (via (at 142.2 140) (size 0.6) (drill 0.3) (layers "F.Cu" "B.Cu") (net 2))
 (via (at 102.2 144) (size 0.6) (drill 0.3) (layers "F.Cu" "B.Cu") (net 2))
 (via (at 106.2 144) (size 0.6) (drill 0.3) (layers "F.Cu" "B.Cu") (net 2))
 (via (at 110.2 144) (size 0.6) (drill 0.3) (layers "F.Cu" "B.Cu") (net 2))
 (via (at 114.2 144) (size 0.6) (drill 0.3) (layers "F.Cu" "B.Cu") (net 2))
 (via (at 118.2 144) (size 0.6) (drill 0.3) (layers "F.Cu" "B.Cu") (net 2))
 (via (at 122.2 144) (size 0.6) (drill 0.3) (layers "F.Cu" "B.Cu") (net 2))
 (via (at 126.2 144) (size 0.6) (drill 0.3) (layers "F.Cu" "B.Cu") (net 2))
 (via (at 130.2 144) (size 0.6) (drill 0.3) (layers "F.Cu" "B.Cu") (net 2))
 (via (at 134.2 144) (size 0.6) (drill 0.3) (layers "F.Cu" "B.Cu") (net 2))
 (via (at 138.2 144) (size 0.6) (drill 0.3) (layers "F.Cu" "B.Cu") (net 2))
 (via (at 142.2 144) (size 0.6) (drill 0.3) (layers "F.Cu" "B.Cu") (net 2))
 (via (at 102.2 148) (size 0.6) (drill 0.3) (layers "F.Cu" "B.Cu") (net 2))
 (via (at 106.2 148) (size 0.6) (drill 0.3) (layers "F.Cu" "B.Cu") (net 2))
 (via (at 110.2 148) (size 0.6) (drill 0.3) (layers "F.Cu" "B.Cu") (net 2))
 (via (at 114.2 148) (size 0.6) (drill 0.3) (layers "F.Cu" "B.Cu") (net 2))
 (via (at 118.2 148) (size 0.6) (drill 0.3) (layers "F.Cu" "B.Cu") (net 2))
 (via (at 122.2 148) (size 0.6) (drill 0.3) (layers "F.Cu" "B.Cu") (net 2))
 (via (at 126.2 148) (size 0.6) (drill 0.3) (layers "F.Cu" "B.Cu") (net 2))
 (via (at 130.2 148) (size 0.6) (drill 0.3) (layers "F.Cu" "B.Cu") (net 2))
 (via (at 134.2 148) (size 0.6) (drill 0.3) (layers "F.Cu" "B.Cu") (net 2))
 (via (at 138.2 148) (size 0.6) (drill 0.3) (layers "F.Cu" "B.Cu") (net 2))
 (via (at 142.2 148) (size 0.6) (drill 0.3) (layers "F.Cu" "B.Cu") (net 2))
 (via (at 102.2 152) (size 0.6) (drill 0.3) (layers "F.Cu" "B.Cu") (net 2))
 (via (at 106.2 152) (size 0.6) (drill 0.3) (layers "F.Cu" "B.Cu") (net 2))
 (via (at 110.2 152) (size 0.6) (drill 0.3) (layers "F.Cu" "B.Cu") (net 2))
 (via (at 114.2 152) (size 0.6) (drill 0.3) (layers "F.Cu" "B.Cu") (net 2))
 (via (at 118.2 152) (size 0.6) (drill 0.3) (layers "F.Cu" "B.Cu") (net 2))
 (via (at 122.2 152) (size 0.6) (drill 0.3) (layers "F.Cu" "B.Cu") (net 2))
 (via (at 126.2 152) (size 0.6) (drill 0.3) (layers "F.Cu" "B.Cu") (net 2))
 (via (at 130.2 152) (size 0.6) (drill 0.3) (layers "F.Cu" "B.Cu") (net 2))
 (via (at 134.2 152) (size 0.6) (drill 0.3) (layers "F.Cu" "B.Cu") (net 2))
 (via (at 138.2 152) (size 0.6) (drill 0.3) (layers "F.Cu" "B.Cu") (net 2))
 (via (at 142.2 152) (size 0.6) (drill 0.3) (layers "F.Cu" "B.Cu") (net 2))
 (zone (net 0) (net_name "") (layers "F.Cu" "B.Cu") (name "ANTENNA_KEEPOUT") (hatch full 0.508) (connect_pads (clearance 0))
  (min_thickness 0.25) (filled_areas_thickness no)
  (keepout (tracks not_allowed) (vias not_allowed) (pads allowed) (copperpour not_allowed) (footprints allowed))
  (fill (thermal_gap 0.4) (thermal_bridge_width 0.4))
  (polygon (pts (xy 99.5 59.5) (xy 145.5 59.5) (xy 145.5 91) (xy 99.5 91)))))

